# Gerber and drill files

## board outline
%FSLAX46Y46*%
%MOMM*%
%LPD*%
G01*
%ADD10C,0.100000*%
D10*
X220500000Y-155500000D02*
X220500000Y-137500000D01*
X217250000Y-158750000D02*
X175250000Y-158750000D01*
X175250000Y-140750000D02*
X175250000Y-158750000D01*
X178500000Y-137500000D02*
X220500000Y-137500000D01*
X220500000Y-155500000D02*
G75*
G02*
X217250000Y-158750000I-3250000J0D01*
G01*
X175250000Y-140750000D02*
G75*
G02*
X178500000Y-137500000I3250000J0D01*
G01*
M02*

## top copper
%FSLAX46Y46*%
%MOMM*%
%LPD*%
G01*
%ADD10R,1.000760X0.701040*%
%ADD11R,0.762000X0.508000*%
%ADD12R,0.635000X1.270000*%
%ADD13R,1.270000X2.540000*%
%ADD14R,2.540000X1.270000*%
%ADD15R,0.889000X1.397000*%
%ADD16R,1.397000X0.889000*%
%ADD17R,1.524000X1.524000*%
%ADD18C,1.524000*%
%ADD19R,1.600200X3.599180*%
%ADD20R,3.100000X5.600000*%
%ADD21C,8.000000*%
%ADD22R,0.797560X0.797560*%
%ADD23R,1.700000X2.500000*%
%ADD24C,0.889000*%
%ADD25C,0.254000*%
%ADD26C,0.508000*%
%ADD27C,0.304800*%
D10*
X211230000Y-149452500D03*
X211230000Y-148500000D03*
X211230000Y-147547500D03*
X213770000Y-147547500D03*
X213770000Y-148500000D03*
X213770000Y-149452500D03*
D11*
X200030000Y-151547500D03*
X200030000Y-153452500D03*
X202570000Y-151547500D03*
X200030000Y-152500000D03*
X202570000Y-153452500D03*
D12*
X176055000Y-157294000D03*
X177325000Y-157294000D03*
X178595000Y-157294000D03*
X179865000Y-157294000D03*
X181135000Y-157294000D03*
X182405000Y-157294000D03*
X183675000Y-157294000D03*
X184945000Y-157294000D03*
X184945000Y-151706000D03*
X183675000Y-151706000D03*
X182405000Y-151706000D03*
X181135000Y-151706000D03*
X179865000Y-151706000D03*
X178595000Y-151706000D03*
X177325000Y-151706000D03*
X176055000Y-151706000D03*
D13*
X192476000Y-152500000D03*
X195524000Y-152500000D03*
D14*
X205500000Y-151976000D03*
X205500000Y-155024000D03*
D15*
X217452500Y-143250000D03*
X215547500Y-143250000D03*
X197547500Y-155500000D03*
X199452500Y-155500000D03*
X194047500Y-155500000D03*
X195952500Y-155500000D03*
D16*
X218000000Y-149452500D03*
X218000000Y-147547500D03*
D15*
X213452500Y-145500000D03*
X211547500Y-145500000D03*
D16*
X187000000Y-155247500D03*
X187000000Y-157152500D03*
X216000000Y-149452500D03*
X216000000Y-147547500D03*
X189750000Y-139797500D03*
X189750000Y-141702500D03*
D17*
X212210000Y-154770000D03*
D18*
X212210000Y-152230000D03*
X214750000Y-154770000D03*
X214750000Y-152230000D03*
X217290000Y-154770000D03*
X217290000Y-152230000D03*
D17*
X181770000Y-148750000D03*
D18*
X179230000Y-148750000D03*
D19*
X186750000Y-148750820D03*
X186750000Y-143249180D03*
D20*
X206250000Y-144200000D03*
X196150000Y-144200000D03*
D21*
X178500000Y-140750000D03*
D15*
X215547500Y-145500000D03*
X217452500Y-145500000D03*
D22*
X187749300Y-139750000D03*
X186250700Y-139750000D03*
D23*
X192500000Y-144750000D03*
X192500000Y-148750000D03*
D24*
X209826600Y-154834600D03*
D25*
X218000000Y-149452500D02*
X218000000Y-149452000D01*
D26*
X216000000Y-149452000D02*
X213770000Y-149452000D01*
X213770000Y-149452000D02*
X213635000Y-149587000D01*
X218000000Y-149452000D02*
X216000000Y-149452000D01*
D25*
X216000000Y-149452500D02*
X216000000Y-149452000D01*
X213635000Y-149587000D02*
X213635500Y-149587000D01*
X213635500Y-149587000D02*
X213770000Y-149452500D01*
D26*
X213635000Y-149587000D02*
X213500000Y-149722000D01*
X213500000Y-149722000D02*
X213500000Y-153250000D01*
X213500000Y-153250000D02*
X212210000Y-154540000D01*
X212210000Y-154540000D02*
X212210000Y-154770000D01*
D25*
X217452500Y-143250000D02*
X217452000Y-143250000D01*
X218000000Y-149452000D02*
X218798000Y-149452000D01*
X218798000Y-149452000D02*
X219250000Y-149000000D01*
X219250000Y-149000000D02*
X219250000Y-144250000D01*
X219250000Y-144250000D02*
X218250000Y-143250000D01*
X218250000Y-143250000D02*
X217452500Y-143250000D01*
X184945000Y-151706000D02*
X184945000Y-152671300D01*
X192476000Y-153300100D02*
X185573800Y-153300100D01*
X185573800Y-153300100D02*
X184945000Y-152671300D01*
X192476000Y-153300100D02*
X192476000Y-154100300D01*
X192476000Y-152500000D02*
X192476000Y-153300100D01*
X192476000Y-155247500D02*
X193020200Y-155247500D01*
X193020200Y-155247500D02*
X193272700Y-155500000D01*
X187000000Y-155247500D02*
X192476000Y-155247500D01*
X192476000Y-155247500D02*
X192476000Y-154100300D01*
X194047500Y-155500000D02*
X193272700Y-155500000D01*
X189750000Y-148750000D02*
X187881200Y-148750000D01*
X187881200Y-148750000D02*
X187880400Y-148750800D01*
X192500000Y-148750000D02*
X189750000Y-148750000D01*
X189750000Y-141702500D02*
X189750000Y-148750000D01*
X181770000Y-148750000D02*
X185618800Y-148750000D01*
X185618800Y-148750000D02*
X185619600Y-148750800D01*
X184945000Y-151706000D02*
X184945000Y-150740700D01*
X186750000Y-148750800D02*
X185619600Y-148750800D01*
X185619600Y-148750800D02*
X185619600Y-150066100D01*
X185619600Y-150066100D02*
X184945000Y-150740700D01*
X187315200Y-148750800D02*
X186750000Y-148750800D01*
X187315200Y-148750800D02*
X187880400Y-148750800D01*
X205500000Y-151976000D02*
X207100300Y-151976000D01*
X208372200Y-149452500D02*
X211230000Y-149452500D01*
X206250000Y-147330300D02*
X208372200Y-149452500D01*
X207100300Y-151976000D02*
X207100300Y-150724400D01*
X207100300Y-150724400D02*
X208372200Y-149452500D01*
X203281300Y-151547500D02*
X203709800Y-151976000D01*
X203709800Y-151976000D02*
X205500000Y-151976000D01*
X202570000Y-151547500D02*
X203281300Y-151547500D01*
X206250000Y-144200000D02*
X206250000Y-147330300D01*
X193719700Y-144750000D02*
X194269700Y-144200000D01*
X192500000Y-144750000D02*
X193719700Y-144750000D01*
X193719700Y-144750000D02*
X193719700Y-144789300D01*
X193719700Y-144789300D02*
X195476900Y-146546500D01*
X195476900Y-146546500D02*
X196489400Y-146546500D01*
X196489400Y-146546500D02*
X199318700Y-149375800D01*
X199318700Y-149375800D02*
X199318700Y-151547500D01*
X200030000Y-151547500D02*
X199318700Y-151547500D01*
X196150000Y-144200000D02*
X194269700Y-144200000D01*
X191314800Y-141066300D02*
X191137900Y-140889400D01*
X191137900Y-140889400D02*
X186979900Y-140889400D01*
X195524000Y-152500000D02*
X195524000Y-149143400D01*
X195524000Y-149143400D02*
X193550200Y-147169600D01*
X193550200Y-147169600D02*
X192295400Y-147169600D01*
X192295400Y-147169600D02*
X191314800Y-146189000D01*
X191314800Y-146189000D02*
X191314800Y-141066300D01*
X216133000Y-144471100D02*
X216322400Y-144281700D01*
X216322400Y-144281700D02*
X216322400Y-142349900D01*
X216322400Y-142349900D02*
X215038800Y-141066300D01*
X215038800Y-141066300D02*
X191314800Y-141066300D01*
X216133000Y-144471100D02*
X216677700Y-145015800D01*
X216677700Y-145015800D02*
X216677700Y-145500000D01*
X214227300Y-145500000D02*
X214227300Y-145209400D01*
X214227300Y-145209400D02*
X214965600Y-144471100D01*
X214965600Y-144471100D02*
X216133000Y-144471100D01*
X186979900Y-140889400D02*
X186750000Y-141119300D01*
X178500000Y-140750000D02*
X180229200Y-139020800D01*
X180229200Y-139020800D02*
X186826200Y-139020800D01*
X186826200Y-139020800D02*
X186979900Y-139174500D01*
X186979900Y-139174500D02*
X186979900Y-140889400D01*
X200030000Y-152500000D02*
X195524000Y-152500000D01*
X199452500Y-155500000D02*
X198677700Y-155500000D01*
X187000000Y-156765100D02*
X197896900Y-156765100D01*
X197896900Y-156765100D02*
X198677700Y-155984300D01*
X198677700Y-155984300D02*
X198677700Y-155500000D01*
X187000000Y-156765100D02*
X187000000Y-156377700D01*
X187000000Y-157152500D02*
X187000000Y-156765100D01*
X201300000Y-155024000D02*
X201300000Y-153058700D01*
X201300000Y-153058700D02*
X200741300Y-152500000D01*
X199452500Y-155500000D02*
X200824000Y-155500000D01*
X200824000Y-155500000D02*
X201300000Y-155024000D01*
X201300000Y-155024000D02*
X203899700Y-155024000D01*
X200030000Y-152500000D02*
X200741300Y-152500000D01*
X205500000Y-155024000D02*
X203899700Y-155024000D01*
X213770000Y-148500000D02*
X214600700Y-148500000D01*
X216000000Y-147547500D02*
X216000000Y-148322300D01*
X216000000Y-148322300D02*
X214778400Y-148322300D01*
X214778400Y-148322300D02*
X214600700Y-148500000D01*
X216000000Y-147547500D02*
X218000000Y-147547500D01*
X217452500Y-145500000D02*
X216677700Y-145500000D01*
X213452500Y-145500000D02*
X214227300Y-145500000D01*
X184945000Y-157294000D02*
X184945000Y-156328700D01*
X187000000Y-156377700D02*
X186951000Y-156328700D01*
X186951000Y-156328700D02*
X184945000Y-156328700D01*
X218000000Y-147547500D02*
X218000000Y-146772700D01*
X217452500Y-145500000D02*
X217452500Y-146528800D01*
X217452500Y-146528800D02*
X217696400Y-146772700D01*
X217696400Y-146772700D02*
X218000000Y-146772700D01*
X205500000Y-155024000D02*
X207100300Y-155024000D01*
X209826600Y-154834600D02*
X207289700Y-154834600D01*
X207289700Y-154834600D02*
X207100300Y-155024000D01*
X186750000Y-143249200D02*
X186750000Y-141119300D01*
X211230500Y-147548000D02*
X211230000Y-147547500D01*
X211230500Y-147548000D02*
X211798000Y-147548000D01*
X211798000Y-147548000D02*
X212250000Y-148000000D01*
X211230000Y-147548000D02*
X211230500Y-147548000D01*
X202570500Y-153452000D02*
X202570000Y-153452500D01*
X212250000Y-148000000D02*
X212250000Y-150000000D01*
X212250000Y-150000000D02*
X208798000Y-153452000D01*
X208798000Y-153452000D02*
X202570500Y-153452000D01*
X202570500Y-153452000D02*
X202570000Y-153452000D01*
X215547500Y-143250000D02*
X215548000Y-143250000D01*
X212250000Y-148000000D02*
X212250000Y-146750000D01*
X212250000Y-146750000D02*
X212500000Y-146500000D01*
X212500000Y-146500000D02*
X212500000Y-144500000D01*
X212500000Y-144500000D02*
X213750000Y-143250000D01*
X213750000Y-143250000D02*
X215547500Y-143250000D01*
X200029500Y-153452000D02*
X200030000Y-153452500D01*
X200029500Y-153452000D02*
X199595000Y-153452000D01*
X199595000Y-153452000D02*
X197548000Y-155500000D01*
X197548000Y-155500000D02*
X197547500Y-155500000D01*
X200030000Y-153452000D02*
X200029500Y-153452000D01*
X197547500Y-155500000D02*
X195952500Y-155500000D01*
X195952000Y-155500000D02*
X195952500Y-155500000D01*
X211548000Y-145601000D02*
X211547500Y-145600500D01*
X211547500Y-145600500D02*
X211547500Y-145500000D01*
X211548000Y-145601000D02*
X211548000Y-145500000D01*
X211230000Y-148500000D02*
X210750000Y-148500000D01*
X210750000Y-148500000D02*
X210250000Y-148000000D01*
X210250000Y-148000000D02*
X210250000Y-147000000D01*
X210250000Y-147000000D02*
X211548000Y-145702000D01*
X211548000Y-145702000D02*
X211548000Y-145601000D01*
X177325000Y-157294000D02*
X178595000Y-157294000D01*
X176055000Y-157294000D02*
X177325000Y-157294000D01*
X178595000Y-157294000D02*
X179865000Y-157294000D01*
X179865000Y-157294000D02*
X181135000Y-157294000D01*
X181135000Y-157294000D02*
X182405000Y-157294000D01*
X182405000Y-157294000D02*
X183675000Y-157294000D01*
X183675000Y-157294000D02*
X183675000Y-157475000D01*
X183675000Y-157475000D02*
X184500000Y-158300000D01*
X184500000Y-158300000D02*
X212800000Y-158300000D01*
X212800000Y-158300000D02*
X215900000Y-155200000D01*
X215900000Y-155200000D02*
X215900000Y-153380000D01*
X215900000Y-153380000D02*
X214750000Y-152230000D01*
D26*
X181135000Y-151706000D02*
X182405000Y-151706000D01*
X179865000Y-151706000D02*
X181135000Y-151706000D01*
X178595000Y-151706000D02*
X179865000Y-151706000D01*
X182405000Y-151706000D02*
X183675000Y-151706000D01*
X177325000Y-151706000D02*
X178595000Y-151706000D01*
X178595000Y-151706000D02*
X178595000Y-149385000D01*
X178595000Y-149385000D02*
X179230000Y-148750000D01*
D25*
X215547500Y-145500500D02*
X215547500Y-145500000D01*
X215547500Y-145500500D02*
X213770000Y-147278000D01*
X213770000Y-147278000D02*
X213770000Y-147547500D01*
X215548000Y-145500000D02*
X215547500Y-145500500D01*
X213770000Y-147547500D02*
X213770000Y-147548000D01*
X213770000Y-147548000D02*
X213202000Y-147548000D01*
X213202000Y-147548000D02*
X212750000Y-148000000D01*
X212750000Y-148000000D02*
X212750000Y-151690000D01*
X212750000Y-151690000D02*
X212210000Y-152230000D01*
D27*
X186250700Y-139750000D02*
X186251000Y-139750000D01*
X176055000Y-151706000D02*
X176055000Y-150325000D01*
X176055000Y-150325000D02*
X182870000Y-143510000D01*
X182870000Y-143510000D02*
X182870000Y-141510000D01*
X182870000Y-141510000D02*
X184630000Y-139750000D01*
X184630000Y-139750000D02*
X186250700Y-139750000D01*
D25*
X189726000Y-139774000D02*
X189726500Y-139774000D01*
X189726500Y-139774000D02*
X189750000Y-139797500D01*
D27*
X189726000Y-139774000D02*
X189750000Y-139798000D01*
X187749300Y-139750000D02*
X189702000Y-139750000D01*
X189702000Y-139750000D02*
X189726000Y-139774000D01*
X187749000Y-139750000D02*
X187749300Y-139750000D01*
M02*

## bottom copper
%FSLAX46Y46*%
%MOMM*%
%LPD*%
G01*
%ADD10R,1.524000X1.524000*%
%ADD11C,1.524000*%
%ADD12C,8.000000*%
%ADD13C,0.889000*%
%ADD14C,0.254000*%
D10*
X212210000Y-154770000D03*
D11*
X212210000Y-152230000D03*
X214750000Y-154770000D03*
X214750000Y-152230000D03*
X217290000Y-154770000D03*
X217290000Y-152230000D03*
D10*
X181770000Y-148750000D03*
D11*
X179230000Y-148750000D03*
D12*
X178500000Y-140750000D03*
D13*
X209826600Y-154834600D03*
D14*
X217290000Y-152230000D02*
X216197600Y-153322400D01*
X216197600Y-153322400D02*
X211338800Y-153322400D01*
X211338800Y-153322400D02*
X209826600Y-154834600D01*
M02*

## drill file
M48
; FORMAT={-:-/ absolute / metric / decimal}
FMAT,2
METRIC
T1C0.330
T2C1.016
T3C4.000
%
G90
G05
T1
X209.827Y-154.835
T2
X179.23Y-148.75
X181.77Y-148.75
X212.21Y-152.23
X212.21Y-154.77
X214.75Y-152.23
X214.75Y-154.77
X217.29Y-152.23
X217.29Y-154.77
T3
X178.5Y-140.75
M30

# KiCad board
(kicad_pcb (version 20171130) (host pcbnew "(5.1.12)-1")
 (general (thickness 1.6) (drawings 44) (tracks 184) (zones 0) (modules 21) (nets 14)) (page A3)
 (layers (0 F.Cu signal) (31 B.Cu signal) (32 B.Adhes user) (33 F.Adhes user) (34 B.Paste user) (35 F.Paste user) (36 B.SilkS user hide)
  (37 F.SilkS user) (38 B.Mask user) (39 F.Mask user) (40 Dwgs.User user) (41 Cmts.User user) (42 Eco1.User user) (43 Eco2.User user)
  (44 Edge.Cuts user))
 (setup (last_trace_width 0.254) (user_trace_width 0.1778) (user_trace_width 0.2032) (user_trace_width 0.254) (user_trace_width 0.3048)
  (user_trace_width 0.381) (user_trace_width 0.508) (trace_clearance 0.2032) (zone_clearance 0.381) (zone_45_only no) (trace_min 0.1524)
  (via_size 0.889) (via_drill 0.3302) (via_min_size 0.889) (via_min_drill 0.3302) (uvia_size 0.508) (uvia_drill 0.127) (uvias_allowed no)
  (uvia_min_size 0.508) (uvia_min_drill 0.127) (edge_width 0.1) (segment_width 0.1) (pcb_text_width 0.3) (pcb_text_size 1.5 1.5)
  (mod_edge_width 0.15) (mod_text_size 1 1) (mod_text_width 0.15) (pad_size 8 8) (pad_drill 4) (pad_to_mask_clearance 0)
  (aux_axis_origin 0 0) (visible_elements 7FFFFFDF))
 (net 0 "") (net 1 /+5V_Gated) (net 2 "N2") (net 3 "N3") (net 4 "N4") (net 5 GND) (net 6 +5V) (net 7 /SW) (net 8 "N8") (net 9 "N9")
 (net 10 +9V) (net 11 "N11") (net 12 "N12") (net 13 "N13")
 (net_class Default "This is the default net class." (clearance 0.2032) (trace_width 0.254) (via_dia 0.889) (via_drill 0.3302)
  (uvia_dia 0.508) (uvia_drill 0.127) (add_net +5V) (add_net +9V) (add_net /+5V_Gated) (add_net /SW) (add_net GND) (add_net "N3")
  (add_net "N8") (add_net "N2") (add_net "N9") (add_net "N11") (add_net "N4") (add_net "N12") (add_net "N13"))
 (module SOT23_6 (layer F.Cu) (at 212.5 148.5 90)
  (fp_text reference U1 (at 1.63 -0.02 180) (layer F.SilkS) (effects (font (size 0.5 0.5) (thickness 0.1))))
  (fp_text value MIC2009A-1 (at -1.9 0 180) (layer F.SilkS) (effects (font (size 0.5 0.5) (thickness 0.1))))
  (pad 6 smd rect (at -0.9525 -1.27 90) (size 0.70104 1.00076) (layers F.Cu F.Paste F.Mask) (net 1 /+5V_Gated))
  (pad 5 smd rect (at 0 -1.27 90) (size 0.70104 1.00076) (layers F.Cu F.Paste F.Mask) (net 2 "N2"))
  (pad 4 smd rect (at 0.9525 -1.27 90) (size 0.70104 1.00076) (layers F.Cu F.Paste F.Mask) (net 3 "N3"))
  (pad 3 smd rect (at 0.9525 1.27 90) (size 0.70104 1.00076) (layers F.Cu F.Paste F.Mask) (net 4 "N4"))
  (pad 2 smd rect (at 0 1.27 90) (size 0.70104 1.00076) (layers F.Cu F.Paste F.Mask) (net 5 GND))
  (pad 1 smd rect (at -0.9525 1.27 90) (size 0.70104 1.00076) (layers F.Cu F.Paste F.Mask) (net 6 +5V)))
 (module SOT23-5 (layer F.Cu) (at 201.3 152.5 270)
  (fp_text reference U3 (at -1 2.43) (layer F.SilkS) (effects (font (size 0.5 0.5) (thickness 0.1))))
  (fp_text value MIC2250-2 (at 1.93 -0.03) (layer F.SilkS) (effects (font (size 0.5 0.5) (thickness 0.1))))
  (pad 1 smd rect (at -0.9525 1.27 270) (size 0.508 0.762) (layers F.Cu F.Paste F.Mask) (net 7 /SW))
  (pad 3 smd rect (at 0.9525 1.27 270) (size 0.508 0.762) (layers F.Cu F.Paste F.Mask) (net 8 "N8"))
  (pad 5 smd rect (at -0.9525 -1.27 270) (size 0.508 0.762) (layers F.Cu F.Paste F.Mask) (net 1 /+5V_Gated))
  (pad 2 smd rect (at 0 1.27 270) (size 0.508 0.762) (layers F.Cu F.Paste F.Mask) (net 5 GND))
  (pad 4 smd rect (at 0.9525 -1.27 270) (size 0.508 0.762) (layers F.Cu F.Paste F.Mask) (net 3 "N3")))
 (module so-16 (layer F.Cu) (at 180.5 154.5)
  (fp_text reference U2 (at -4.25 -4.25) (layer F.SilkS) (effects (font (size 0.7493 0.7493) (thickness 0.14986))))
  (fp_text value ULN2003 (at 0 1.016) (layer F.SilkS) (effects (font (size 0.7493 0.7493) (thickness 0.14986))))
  (pad 1 smd rect (at -4.445 2.794) (size 0.635 1.27) (layers F.Cu F.Paste F.Mask) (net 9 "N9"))
  (pad 2 smd rect (at -3.175 2.794) (size 0.635 1.27) (layers F.Cu F.Paste F.Mask) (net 9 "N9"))
  (pad 3 smd rect (at -1.905 2.794) (size 0.635 1.27) (layers F.Cu F.Paste F.Mask) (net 9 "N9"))
  (pad 4 smd rect (at -0.635 2.794) (size 0.635 1.27) (layers F.Cu F.Paste F.Mask) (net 9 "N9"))
  (pad 5 smd rect (at 0.635 2.794) (size 0.635 1.27) (layers F.Cu F.Paste F.Mask) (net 9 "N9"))
  (pad 6 smd rect (at 1.905 2.794) (size 0.635 1.27) (layers F.Cu F.Paste F.Mask) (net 9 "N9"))
  (pad 7 smd rect (at 3.175 2.794) (size 0.635 1.27) (layers F.Cu F.Paste F.Mask) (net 9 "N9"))
  (pad 8 smd rect (at 4.445 2.794) (size 0.635 1.27) (layers F.Cu F.Paste F.Mask) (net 5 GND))
  (pad 9 smd rect (at 4.445 -2.794) (size 0.635 1.27) (layers F.Cu F.Paste F.Mask) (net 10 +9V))
  (pad 10 smd rect (at 3.175 -2.794) (size 0.635 1.27) (layers F.Cu F.Paste F.Mask) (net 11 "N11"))
  (pad 11 smd rect (at 1.905 -2.794) (size 0.635 1.27) (layers F.Cu F.Paste F.Mask) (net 11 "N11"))
  (pad 12 smd rect (at 0.635 -2.794) (size 0.635 1.27) (layers F.Cu F.Paste F.Mask) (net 11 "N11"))
  (pad 13 smd rect (at -0.635 -2.794) (size 0.635 1.27) (layers F.Cu F.Paste F.Mask) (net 11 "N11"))
  (pad 14 smd rect (at -1.905 -2.794) (size 0.635 1.27) (layers F.Cu F.Paste F.Mask) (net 11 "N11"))
  (pad 15 smd rect (at -3.175 -2.794) (size 0.635 1.27) (layers F.Cu F.Paste F.Mask) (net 11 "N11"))
  (pad 16 smd rect (at -4.445 -2.794) (size 0.635 1.27) (layers F.Cu F.Paste F.Mask) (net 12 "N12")))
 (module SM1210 (layer F.Cu) (at 194 152.5)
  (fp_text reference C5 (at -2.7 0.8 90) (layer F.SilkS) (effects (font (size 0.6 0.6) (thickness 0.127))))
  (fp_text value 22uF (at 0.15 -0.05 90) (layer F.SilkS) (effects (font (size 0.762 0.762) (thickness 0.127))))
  (pad 1 smd rect (at -1.524 0) (size 1.27 2.54) (layers F.Cu F.Paste F.Mask) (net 10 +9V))
  (pad 2 smd rect (at 1.524 0) (size 1.27 2.54) (layers F.Cu F.Paste F.Mask) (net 5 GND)))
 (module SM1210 (layer F.Cu) (at 205.5 153.5 270)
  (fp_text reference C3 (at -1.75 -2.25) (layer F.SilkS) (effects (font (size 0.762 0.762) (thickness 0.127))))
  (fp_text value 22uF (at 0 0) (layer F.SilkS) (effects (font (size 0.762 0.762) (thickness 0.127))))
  (pad 1 smd rect (at -1.524 0 270) (size 1.27 2.54) (layers F.Cu F.Paste F.Mask) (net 1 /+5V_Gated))
  (pad 2 smd rect (at 1.524 0 270) (size 1.27 2.54) (layers F.Cu F.Paste F.Mask) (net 5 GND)))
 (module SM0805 (layer F.Cu) (at 216.5 143.25 180)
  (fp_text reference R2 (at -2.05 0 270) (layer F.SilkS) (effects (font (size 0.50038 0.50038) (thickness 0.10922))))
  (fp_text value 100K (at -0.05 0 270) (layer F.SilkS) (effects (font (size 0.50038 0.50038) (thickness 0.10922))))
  (pad 1 smd rect (at -0.9525 0 180) (size 0.889 1.397) (layers F.Cu F.Paste F.Mask) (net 6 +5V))
  (pad 2 smd rect (at 0.9525 0 180) (size 0.889 1.397) (layers F.Cu F.Paste F.Mask) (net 3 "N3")))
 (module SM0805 (layer F.Cu) (at 198.5 155.5)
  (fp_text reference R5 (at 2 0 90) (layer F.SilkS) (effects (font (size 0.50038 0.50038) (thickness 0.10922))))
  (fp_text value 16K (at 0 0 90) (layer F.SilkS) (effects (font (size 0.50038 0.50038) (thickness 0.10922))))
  (pad 1 smd rect (at -0.9525 0) (size 0.889 1.397) (layers F.Cu F.Paste F.Mask) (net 8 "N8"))
  (pad 2 smd rect (at 0.9525 0) (size 0.889 1.397) (layers F.Cu F.Paste F.Mask) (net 5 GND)))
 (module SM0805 (layer F.Cu) (at 195 155.5)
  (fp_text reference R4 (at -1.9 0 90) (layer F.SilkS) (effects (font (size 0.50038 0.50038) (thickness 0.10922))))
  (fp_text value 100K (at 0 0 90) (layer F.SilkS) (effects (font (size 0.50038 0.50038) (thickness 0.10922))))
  (pad 1 smd rect (at -0.9525 0) (size 0.889 1.397) (layers F.Cu F.Paste F.Mask) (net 10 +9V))
  (pad 2 smd rect (at 0.9525 0) (size 0.889 1.397) (layers F.Cu F.Paste F.Mask) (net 8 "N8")))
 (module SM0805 (layer F.Cu) (at 218 148.5 90)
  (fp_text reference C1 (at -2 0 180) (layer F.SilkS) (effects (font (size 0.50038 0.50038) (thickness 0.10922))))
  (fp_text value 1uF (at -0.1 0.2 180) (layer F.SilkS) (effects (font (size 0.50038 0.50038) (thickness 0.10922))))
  (pad 1 smd rect (at -0.9525 0 90) (size 0.889 1.397) (layers F.Cu F.Paste F.Mask) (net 6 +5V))
  (pad 2 smd rect (at 0.9525 0 90) (size 0.889 1.397) (layers F.Cu F.Paste F.Mask) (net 5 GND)))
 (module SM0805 (layer F.Cu) (at 212.5 145.5 180)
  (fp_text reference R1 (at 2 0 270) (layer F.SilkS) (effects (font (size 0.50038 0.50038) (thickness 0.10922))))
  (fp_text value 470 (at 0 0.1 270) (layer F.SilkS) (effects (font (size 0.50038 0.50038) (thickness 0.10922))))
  (pad 1 smd rect (at -0.9525 0 180) (size 0.889 1.397) (layers F.Cu F.Paste F.Mask) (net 5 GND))
  (pad 2 smd rect (at 0.9525 0 180) (size 0.889 1.397) (layers F.Cu F.Paste F.Mask) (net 2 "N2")))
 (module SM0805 (layer F.Cu) (at 187 156.2 270)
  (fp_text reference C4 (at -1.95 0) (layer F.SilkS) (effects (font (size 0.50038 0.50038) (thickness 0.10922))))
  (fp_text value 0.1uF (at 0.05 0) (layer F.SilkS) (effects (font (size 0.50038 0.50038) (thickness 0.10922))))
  (pad 1 smd rect (at -0.9525 0 270) (size 0.889 1.397) (layers F.Cu F.Paste F.Mask) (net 10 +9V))
  (pad 2 smd rect (at 0.9525 0 270) (size 0.889 1.397) (layers F.Cu F.Paste F.Mask) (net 5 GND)))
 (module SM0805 (layer F.Cu) (at 216 148.5 90)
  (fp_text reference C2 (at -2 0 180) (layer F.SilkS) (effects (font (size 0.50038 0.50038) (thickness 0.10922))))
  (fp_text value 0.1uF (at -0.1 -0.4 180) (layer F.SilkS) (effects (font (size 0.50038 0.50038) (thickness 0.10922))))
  (pad 1 smd rect (at -0.9525 0 90) (size 0.889 1.397) (layers F.Cu F.Paste F.Mask) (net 6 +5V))
  (pad 2 smd rect (at 0.9525 0 90) (size 0.889 1.397) (layers F.Cu F.Paste F.Mask) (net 5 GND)))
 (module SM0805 (layer F.Cu) (at 189.75 140.75 270)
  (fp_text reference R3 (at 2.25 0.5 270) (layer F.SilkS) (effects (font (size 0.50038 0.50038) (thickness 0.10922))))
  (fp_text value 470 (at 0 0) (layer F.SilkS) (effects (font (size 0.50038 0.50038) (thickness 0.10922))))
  (pad 1 smd rect (at -0.9525 0 270) (size 0.889 1.397) (layers F.Cu F.Paste F.Mask) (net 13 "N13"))
  (pad 2 smd rect (at 0.9525 0 270) (size 0.889 1.397) (layers F.Cu F.Paste F.Mask) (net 10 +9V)))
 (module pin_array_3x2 (layer F.Cu) (at 214.75 153.5)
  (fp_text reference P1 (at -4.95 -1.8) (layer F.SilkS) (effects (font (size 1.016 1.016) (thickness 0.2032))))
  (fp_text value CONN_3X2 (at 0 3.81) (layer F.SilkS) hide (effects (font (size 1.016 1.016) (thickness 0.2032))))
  (pad 1 thru_hole rect (at -2.54 1.27) (size 1.524 1.524) (drill 1.016) (layers *.Cu *.Mask F.SilkS) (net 6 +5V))
  (pad 2 thru_hole circle (at -2.54 -1.27) (size 1.524 1.524) (drill 1.016) (layers *.Cu *.Mask F.SilkS) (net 4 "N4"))
  (pad 3 thru_hole circle (at 0 1.27) (size 1.524 1.524) (drill 1.016) (layers *.Cu *.Mask F.SilkS))
  (pad 4 thru_hole circle (at 0 -1.27) (size 1.524 1.524) (drill 1.016) (layers *.Cu *.Mask F.SilkS) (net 9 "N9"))
  (pad 5 thru_hole circle (at 2.54 1.27) (size 1.524 1.524) (drill 1.016) (layers *.Cu *.Mask F.SilkS))
  (pad 6 thru_hole circle (at 2.54 -1.27) (size 1.524 1.524) (drill 1.016) (layers *.Cu *.Mask F.SilkS) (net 5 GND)))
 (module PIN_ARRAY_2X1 (layer F.Cu) (at 180.5 148.75 180)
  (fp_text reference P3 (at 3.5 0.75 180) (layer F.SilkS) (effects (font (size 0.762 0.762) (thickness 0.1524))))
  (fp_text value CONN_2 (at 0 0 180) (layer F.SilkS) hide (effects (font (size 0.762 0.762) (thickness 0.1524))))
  (pad 1 thru_hole rect (at -1.27 0 180) (size 1.524 1.524) (drill 1.016) (layers *.Cu *.Mask F.SilkS) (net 10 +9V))
  (pad 2 thru_hole circle (at 1.27 0 180) (size 1.524 1.524) (drill 1.016) (layers *.Cu *.Mask F.SilkS) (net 11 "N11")))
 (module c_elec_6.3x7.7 (layer F.Cu) (at 186.75 146 270)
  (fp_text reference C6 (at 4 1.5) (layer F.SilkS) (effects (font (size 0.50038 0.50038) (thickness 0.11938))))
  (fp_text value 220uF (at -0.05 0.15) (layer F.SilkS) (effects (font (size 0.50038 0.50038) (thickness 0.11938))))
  (pad 1 smd rect (at 2.75082 0 270) (size 3.59918 1.6002) (layers F.Cu F.Paste F.Mask) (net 10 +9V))
  (pad 2 smd rect (at -2.75082 0 270) (size 3.59918 1.6002) (layers F.Cu F.Paste F.Mask) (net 5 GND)))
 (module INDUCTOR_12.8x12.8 (layer F.Cu) (at 201.2 144.2 180)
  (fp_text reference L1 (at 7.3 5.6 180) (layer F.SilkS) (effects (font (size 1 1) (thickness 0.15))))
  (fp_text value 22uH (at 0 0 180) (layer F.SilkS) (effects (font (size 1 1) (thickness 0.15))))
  (pad 1 smd rect (at -5.05 0 180) (size 3.1 5.6) (layers F.Cu F.Paste F.Mask) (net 1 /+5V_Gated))
  (pad 2 smd rect (at 5.05 0 180) (size 3.1 5.6) (layers F.Cu F.Paste F.Mask) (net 7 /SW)))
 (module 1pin (layer F.Cu) (at 178.5 140.75)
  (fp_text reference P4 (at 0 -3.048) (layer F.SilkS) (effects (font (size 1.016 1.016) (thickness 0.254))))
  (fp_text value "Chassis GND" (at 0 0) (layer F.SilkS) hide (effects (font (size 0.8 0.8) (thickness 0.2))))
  (pad 1 thru_hole circle (at 0 0) (size 8 8) (drill 4) (layers *.Cu *.Mask F.SilkS) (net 5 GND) (zone_connect 2)))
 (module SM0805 (layer F.Cu) (at 216.5 145.5)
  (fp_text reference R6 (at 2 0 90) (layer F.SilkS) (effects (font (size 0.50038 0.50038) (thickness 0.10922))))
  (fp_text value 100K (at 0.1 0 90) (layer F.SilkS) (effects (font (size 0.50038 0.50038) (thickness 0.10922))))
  (pad 1 smd rect (at -0.9525 0) (size 0.889 1.397) (layers F.Cu F.Paste F.Mask) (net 4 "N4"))
  (pad 2 smd rect (at 0.9525 0) (size 0.889 1.397) (layers F.Cu F.Paste F.Mask) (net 5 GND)))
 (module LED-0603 (layer F.Cu) (at 187 139.75 180)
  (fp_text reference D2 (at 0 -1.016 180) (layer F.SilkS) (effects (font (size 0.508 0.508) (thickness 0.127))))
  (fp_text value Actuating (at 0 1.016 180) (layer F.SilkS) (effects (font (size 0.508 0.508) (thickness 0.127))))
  (pad 1 smd rect (at -0.7493 0 180) (size 0.79756 0.79756) (layers F.Cu F.Paste F.Mask) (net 13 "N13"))
  (pad 2 smd rect (at 0.7493 0 180) (size 0.79756 0.79756) (layers F.Cu F.Paste F.Mask) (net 12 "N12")))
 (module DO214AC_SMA (layer F.Cu) (at 192.5 146.75 270)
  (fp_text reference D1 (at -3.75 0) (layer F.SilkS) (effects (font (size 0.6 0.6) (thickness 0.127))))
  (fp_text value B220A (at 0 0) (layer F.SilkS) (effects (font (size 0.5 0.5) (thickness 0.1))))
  (pad 1 smd rect (at -2 0 270) (size 2.5 1.7) (layers F.Cu F.Paste F.Mask) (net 7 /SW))
  (pad 2 smd rect (at 2 0 270) (size 2.5 1.7) (layers F.Cu F.Paste F.Mask) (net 10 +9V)))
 (gr_line (start 220.5 155.5) (end 220.5 137.5) (angle 90) (layer Edge.Cuts) (width 0.1))
 (gr_line (start 217.25 158.75) (end 175.25 158.75) (angle 90) (layer Edge.Cuts) (width 0.1))
 (gr_line (start 175.25 140.75) (end 175.25 158.75) (angle 90) (layer Edge.Cuts) (width 0.1))
 (gr_line (start 178.5 137.5) (end 220.5 137.5) (angle 90) (layer Edge.Cuts) (width 0.1))
 (gr_arc (start 217.25 155.5) (end 220.5 155.5) (angle 90) (layer Edge.Cuts) (width 0.1))
 (gr_arc (start 178.5 140.75) (end 175.25 140.75) (angle 90) (layer Edge.Cuts) (width 0.1))
 (segment (start 218 149.4525) (end 218 149.452) (width 0.254) (layer F.Cu) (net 6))
 (segment (start 216 149.452) (end 213.77 149.452) (width 0.508) (layer F.Cu) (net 6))
 (segment (start 213.77 149.452) (end 213.635 149.587) (width 0.508) (layer F.Cu) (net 6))
 (segment (start 218 149.452) (end 216 149.452) (width 0.508) (layer F.Cu) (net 6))
 (segment (start 216 149.4525) (end 216 149.452) (width 0.254) (layer F.Cu) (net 6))
 (segment (start 213.635 149.587) (end 213.6355 149.587) (width 0.254) (layer F.Cu) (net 6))
 (segment (start 213.6355 149.587) (end 213.77 149.4525) (width 0.254) (layer F.Cu) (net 6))
 (segment (start 213.635 149.587) (end 213.5 149.722) (width 0.508) (layer F.Cu) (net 6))
 (segment (start 213.5 149.722) (end 213.5 153.25) (width 0.508) (layer F.Cu) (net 6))
 (segment (start 213.5 153.25) (end 212.21 154.54) (width 0.508) (layer F.Cu) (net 6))
 (segment (start 212.21 154.54) (end 212.21 154.77) (width 0.508) (layer F.Cu) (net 6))
 (segment (start 217.4525 143.25) (end 217.452 143.25) (width 0.254) (layer F.Cu) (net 6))
 (segment (start 218 149.452) (end 218.798 149.452) (width 0.254) (layer F.Cu) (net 6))
 (segment (start 218.798 149.452) (end 219.25 149) (width 0.254) (layer F.Cu) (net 6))
 (segment (start 219.25 149) (end 219.25 144.25) (width 0.254) (layer F.Cu) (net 6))
 (segment (start 219.25 144.25) (end 218.25 143.25) (width 0.254) (layer F.Cu) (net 6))
 (segment (start 218.25 143.25) (end 217.4525 143.25) (width 0.254) (layer F.Cu) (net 6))
 (segment (start 184.945 151.706) (end 184.945 152.6713) (width 0.254) (layer F.Cu) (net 10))
 (segment (start 192.476 153.3001) (end 185.5738 153.3001) (width 0.254) (layer F.Cu) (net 10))
 (segment (start 185.5738 153.3001) (end 184.945 152.6713) (width 0.254) (layer F.Cu) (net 10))
 (segment (start 192.476 153.3001) (end 192.476 154.1003) (width 0.254) (layer F.Cu) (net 10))
 (segment (start 192.476 152.5) (end 192.476 153.3001) (width 0.254) (layer F.Cu) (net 10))
 (segment (start 192.476 155.2475) (end 193.0202 155.2475) (width 0.254) (layer F.Cu) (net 10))
 (segment (start 193.0202 155.2475) (end 193.2727 155.5) (width 0.254) (layer F.Cu) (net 10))
 (segment (start 187 155.2475) (end 192.476 155.2475) (width 0.254) (layer F.Cu) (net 10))
 (segment (start 192.476 155.2475) (end 192.476 154.1003) (width 0.254) (layer F.Cu) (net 10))
 (segment (start 194.0475 155.5) (end 193.2727 155.5) (width 0.254) (layer F.Cu) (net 10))
 (segment (start 189.75 148.75) (end 187.8812 148.75) (width 0.254) (layer F.Cu) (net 10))
 (segment (start 187.8812 148.75) (end 187.8804 148.7508) (width 0.254) (layer F.Cu) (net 10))
 (segment (start 192.5 148.75) (end 189.75 148.75) (width 0.254) (layer F.Cu) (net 10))
 (segment (start 189.75 141.7025) (end 189.75 148.75) (width 0.254) (layer F.Cu) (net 10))
 (segment (start 181.77 148.75) (end 185.6188 148.75) (width 0.254) (layer F.Cu) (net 10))
 (segment (start 185.6188 148.75) (end 185.6196 148.7508) (width 0.254) (layer F.Cu) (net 10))
 (segment (start 184.945 151.706) (end 184.945 150.7407) (width 0.254) (layer F.Cu) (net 10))
 (segment (start 186.75 148.7508) (end 185.6196 148.7508) (width 0.254) (layer F.Cu) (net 10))
 (segment (start 185.6196 148.7508) (end 185.6196 150.0661) (width 0.254) (layer F.Cu) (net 10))
 (segment (start 185.6196 150.0661) (end 184.945 150.7407) (width 0.254) (layer F.Cu) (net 10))
 (segment (start 187.3152 148.7508) (end 186.75 148.7508) (width 0.254) (layer F.Cu) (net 10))
 (segment (start 187.3152 148.7508) (end 187.8804 148.7508) (width 0.254) (layer F.Cu) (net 10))
 (segment (start 205.5 151.976) (end 207.1003 151.976) (width 0.254) (layer F.Cu) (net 1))
 (segment (start 208.3722 149.4525) (end 211.23 149.4525) (width 0.254) (layer F.Cu) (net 1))
 (segment (start 206.25 147.3303) (end 208.3722 149.4525) (width 0.254) (layer F.Cu) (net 1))
 (segment (start 207.1003 151.976) (end 207.1003 150.7244) (width 0.254) (layer F.Cu) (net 1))
 (segment (start 207.1003 150.7244) (end 208.3722 149.4525) (width 0.254) (layer F.Cu) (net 1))
 (segment (start 203.2813 151.5475) (end 203.7098 151.976) (width 0.254) (layer F.Cu) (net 1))
 (segment (start 203.7098 151.976) (end 205.5 151.976) (width 0.254) (layer F.Cu) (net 1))
 (segment (start 202.57 151.5475) (end 203.2813 151.5475) (width 0.254) (layer F.Cu) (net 1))
 (segment (start 206.25 144.2) (end 206.25 147.3303) (width 0.254) (layer F.Cu) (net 1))
 (segment (start 193.7197 144.75) (end 194.2697 144.2) (width 0.254) (layer F.Cu) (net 7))
 (segment (start 192.5 144.75) (end 193.7197 144.75) (width 0.254) (layer F.Cu) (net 7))
 (segment (start 193.7197 144.75) (end 193.7197 144.7893) (width 0.254) (layer F.Cu) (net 7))
 (segment (start 193.7197 144.7893) (end 195.4769 146.5465) (width 0.254) (layer F.Cu) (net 7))
 (segment (start 195.4769 146.5465) (end 196.4894 146.5465) (width 0.254) (layer F.Cu) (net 7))
 (segment (start 196.4894 146.5465) (end 199.3187 149.3758) (width 0.254) (layer F.Cu) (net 7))
 (segment (start 199.3187 149.3758) (end 199.3187 151.5475) (width 0.254) (layer F.Cu) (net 7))
 (segment (start 200.03 151.5475) (end 199.3187 151.5475) (width 0.254) (layer F.Cu) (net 7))
 (segment (start 196.15 144.2) (end 194.2697 144.2) (width 0.254) (layer F.Cu) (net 7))
 (segment (start 191.3148 141.0663) (end 191.1379 140.8894) (width 0.254) (layer F.Cu) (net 5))
 (segment (start 191.1379 140.8894) (end 186.9799 140.8894) (width 0.254) (layer F.Cu) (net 5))
 (segment (start 195.524 152.5) (end 195.524 149.1434) (width 0.254) (layer F.Cu) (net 5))
 (segment (start 195.524 149.1434) (end 193.5502 147.1696) (width 0.254) (layer F.Cu) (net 5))
 (segment (start 193.5502 147.1696) (end 192.2954 147.1696) (width 0.254) (layer F.Cu) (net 5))
 (segment (start 192.2954 147.1696) (end 191.3148 146.189) (width 0.254) (layer F.Cu) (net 5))
 (segment (start 191.3148 146.189) (end 191.3148 141.0663) (width 0.254) (layer F.Cu) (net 5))
 (segment (start 216.133 144.4711) (end 216.3224 144.2817) (width 0.254) (layer F.Cu) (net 5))
 (segment (start 216.3224 144.2817) (end 216.3224 142.3499) (width 0.254) (layer F.Cu) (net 5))
 (segment (start 216.3224 142.3499) (end 215.0388 141.0663) (width 0.254) (layer F.Cu) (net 5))
 (segment (start 215.0388 141.0663) (end 191.3148 141.0663) (width 0.254) (layer F.Cu) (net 5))
 (segment (start 216.133 144.4711) (end 216.6777 145.0158) (width 0.254) (layer F.Cu) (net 5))
 (segment (start 216.6777 145.0158) (end 216.6777 145.5) (width 0.254) (layer F.Cu) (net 5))
 (segment (start 214.2273 145.5) (end 214.2273 145.2094) (width 0.254) (layer F.Cu) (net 5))
 (segment (start 214.2273 145.2094) (end 214.9656 144.4711) (width 0.254) (layer F.Cu) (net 5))
 (segment (start 214.9656 144.4711) (end 216.133 144.4711) (width 0.254) (layer F.Cu) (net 5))
 (segment (start 186.9799 140.8894) (end 186.75 141.1193) (width 0.254) (layer F.Cu) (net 5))
 (segment (start 178.5 140.75) (end 180.2292 139.0208) (width 0.254) (layer F.Cu) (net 5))
 (segment (start 180.2292 139.0208) (end 186.8262 139.0208) (width 0.254) (layer F.Cu) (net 5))
 (segment (start 186.8262 139.0208) (end 186.9799 139.1745) (width 0.254) (layer F.Cu) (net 5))
 (segment (start 186.9799 139.1745) (end 186.9799 140.8894) (width 0.254) (layer F.Cu) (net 5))
 (segment (start 200.03 152.5) (end 195.524 152.5) (width 0.254) (layer F.Cu) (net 5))
 (segment (start 199.4525 155.5) (end 198.6777 155.5) (width 0.254) (layer F.Cu) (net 5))
 (segment (start 187 156.7651) (end 197.8969 156.7651) (width 0.254) (layer F.Cu) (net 5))
 (segment (start 197.8969 156.7651) (end 198.6777 155.9843) (width 0.254) (layer F.Cu) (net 5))
 (segment (start 198.6777 155.9843) (end 198.6777 155.5) (width 0.254) (layer F.Cu) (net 5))
 (segment (start 187 156.7651) (end 187 156.3777) (width 0.254) (layer F.Cu) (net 5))
 (segment (start 187 157.1525) (end 187 156.7651) (width 0.254) (layer F.Cu) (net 5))
 (segment (start 201.3 155.024) (end 201.3 153.0587) (width 0.254) (layer F.Cu) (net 5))
 (segment (start 201.3 153.0587) (end 200.7413 152.5) (width 0.254) (layer F.Cu) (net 5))
 (segment (start 199.4525 155.5) (end 200.824 155.5) (width 0.254) (layer F.Cu) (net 5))
 (segment (start 200.824 155.5) (end 201.3 155.024) (width 0.254) (layer F.Cu) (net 5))
 (segment (start 201.3 155.024) (end 203.8997 155.024) (width 0.254) (layer F.Cu) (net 5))
 (segment (start 200.03 152.5) (end 200.7413 152.5) (width 0.254) (layer F.Cu) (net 5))
 (segment (start 205.5 155.024) (end 203.8997 155.024) (width 0.254) (layer F.Cu) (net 5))
 (segment (start 213.77 148.5) (end 214.6007 148.5) (width 0.254) (layer F.Cu) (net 5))
 (segment (start 216 147.5475) (end 216 148.3223) (width 0.254) (layer F.Cu) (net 5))
 (segment (start 216 148.3223) (end 214.7784 148.3223) (width 0.254) (layer F.Cu) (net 5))
 (segment (start 214.7784 148.3223) (end 214.6007 148.5) (width 0.254) (layer F.Cu) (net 5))
 (segment (start 216 147.5475) (end 218 147.5475) (width 0.254) (layer F.Cu) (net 5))
 (segment (start 217.4525 145.5) (end 216.6777 145.5) (width 0.254) (layer F.Cu) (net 5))
 (segment (start 213.4525 145.5) (end 214.2273 145.5) (width 0.254) (layer F.Cu) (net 5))
 (segment (start 184.945 157.294) (end 184.945 156.3287) (width 0.254) (layer F.Cu) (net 5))
 (segment (start 187 156.3777) (end 186.951 156.3287) (width 0.254) (layer F.Cu) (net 5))
 (segment (start 186.951 156.3287) (end 184.945 156.3287) (width 0.254) (layer F.Cu) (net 5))
 (segment (start 218 147.5475) (end 218 146.7727) (width 0.254) (layer F.Cu) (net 5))
 (segment (start 217.4525 145.5) (end 217.4525 146.5288) (width 0.254) (layer F.Cu) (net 5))
 (segment (start 217.4525 146.5288) (end 217.6964 146.7727) (width 0.254) (layer F.Cu) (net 5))
 (segment (start 217.6964 146.7727) (end 218 146.7727) (width 0.254) (layer F.Cu) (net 5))
 (segment (start 205.5 155.024) (end 207.1003 155.024) (width 0.254) (layer F.Cu) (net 5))
 (segment (start 209.8266 154.8346) (end 207.2897 154.8346) (width 0.254) (layer F.Cu) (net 5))
 (segment (start 207.2897 154.8346) (end 207.1003 155.024) (width 0.254) (layer F.Cu) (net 5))
 (segment (start 217.29 152.23) (end 216.1976 153.3224) (width 0.254) (layer B.Cu) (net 5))
 (segment (start 216.1976 153.3224) (end 211.3388 153.3224) (width 0.254) (layer B.Cu) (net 5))
 (segment (start 211.3388 153.3224) (end 209.8266 154.8346) (width 0.254) (layer B.Cu) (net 5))
 (segment (start 186.75 143.2492) (end 186.75 141.1193) (width 0.254) (layer F.Cu) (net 5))
 (via (at 209.8266 154.8346) (size 0.889) (layers F.Cu B.Cu) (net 5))
 (segment (start 211.2305 147.548) (end 211.23 147.5475) (width 0.254) (layer F.Cu) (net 3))
 (segment (start 211.2305 147.548) (end 211.798 147.548) (width 0.254) (layer F.Cu) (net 3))
 (segment (start 211.798 147.548) (end 212.25 148) (width 0.254) (layer F.Cu) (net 3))
 (segment (start 211.23 147.548) (end 211.2305 147.548) (width 0.254) (layer F.Cu) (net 3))
 (segment (start 202.5705 153.452) (end 202.57 153.4525) (width 0.254) (layer F.Cu) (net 3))
 (segment (start 212.25 148) (end 212.25 150) (width 0.254) (layer F.Cu) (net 3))
 (segment (start 212.25 150) (end 208.798 153.452) (width 0.254) (layer F.Cu) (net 3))
 (segment (start 208.798 153.452) (end 202.5705 153.452) (width 0.254) (layer F.Cu) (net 3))
 (segment (start 202.5705 153.452) (end 202.57 153.452) (width 0.254) (layer F.Cu) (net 3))
 (segment (start 215.5475 143.25) (end 215.548 143.25) (width 0.254) (layer F.Cu) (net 3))
 (segment (start 212.25 148) (end 212.25 146.75) (width 0.254) (layer F.Cu) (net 3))
 (segment (start 212.25 146.75) (end 212.5 146.5) (width 0.254) (layer F.Cu) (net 3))
 (segment (start 212.5 146.5) (end 212.5 144.5) (width 0.254) (layer F.Cu) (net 3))
 (segment (start 212.5 144.5) (end 213.75 143.25) (width 0.254) (layer F.Cu) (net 3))
 (segment (start 213.75 143.25) (end 215.5475 143.25) (width 0.254) (layer F.Cu) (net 3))
 (segment (start 200.0295 153.452) (end 200.03 153.4525) (width 0.254) (layer F.Cu) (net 8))
 (segment (start 200.0295 153.452) (end 199.595 153.452) (width 0.254) (layer F.Cu) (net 8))
 (segment (start 199.595 153.452) (end 197.548 155.5) (width 0.254) (layer F.Cu) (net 8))
 (segment (start 197.548 155.5) (end 197.5475 155.5) (width 0.254) (layer F.Cu) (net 8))
 (segment (start 200.03 153.452) (end 200.0295 153.452) (width 0.254) (layer F.Cu) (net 8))
 (segment (start 197.5475 155.5) (end 195.9525 155.5) (width 0.254) (layer F.Cu) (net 8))
 (segment (start 195.952 155.5) (end 195.9525 155.5) (width 0.254) (layer F.Cu) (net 8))
 (segment (start 211.548 145.601) (end 211.5475 145.6005) (width 0.254) (layer F.Cu) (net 2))
 (segment (start 211.5475 145.6005) (end 211.5475 145.5) (width 0.254) (layer F.Cu) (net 2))
 (segment (start 211.548 145.601) (end 211.548 145.5) (width 0.254) (layer F.Cu) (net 2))
 (segment (start 211.23 148.5) (end 210.75 148.5) (width 0.254) (layer F.Cu) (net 2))
 (segment (start 210.75 148.5) (end 210.25 148) (width 0.254) (layer F.Cu) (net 2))
 (segment (start 210.25 148) (end 210.25 147) (width 0.254) (layer F.Cu) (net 2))
 (segment (start 210.25 147) (end 211.548 145.702) (width 0.254) (layer F.Cu) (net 2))
 (segment (start 211.548 145.702) (end 211.548 145.601) (width 0.254) (layer F.Cu) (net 2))
 (segment (start 177.325 157.294) (end 178.595 157.294) (width 0.254) (layer F.Cu) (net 9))
 (segment (start 176.055 157.294) (end 177.325 157.294) (width 0.254) (layer F.Cu) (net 9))
 (segment (start 178.595 157.294) (end 179.865 157.294) (width 0.254) (layer F.Cu) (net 9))
 (segment (start 179.865 157.294) (end 181.135 157.294) (width 0.254) (layer F.Cu) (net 9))
 (segment (start 181.135 157.294) (end 182.405 157.294) (width 0.254) (layer F.Cu) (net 9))
 (segment (start 182.405 157.294) (end 183.675 157.294) (width 0.254) (layer F.Cu) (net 9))
 (segment (start 183.675 157.294) (end 183.675 157.475) (width 0.254) (layer F.Cu) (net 9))
 (segment (start 183.675 157.475) (end 184.5 158.3) (width 0.254) (layer F.Cu) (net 9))
 (segment (start 184.5 158.3) (end 212.8 158.3) (width 0.254) (layer F.Cu) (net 9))
 (segment (start 212.8 158.3) (end 215.9 155.2) (width 0.254) (layer F.Cu) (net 9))
 (segment (start 215.9 155.2) (end 215.9 153.38) (width 0.254) (layer F.Cu) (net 9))
 (segment (start 215.9 153.38) (end 214.75 152.23) (width 0.254) (layer F.Cu) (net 9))
 (segment (start 181.135 151.706) (end 182.405 151.706) (width 0.508) (layer F.Cu) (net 11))
 (segment (start 179.865 151.706) (end 181.135 151.706) (width 0.508) (layer F.Cu) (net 11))
 (segment (start 178.595 151.706) (end 179.865 151.706) (width 0.508) (layer F.Cu) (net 11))
 (segment (start 182.405 151.706) (end 183.675 151.706) (width 0.508) (layer F.Cu) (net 11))
 (segment (start 177.325 151.706) (end 178.595 151.706) (width 0.508) (layer F.Cu) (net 11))
 (segment (start 178.595 151.706) (end 178.595 149.385) (width 0.508) (layer F.Cu) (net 11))
 (segment (start 178.595 149.385) (end 179.23 148.75) (width 0.508) (layer F.Cu) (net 11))
 (segment (start 215.5475 145.5005) (end 215.5475 145.5) (width 0.254) (layer F.Cu) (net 4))
 (segment (start 215.5475 145.5005) (end 213.77 147.278) (width 0.254) (layer F.Cu) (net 4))
 (segment (start 213.77 147.278) (end 213.77 147.5475) (width 0.254) (layer F.Cu) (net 4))
 (segment (start 215.548 145.5) (end 215.5475 145.5005) (width 0.254) (layer F.Cu) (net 4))
 (segment (start 213.77 147.5475) (end 213.77 147.548) (width 0.254) (layer F.Cu) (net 4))
 (segment (start 213.77 147.548) (end 213.202 147.548) (width 0.254) (layer F.Cu) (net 4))
 (segment (start 213.202 147.548) (end 212.75 148) (width 0.254) (layer F.Cu) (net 4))
 (segment (start 212.75 148) (end 212.75 151.69) (width 0.254) (layer F.Cu) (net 4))
 (segment (start 212.75 151.69) (end 212.21 152.23) (width 0.254) (layer F.Cu) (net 4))
 (segment (start 186.2507 139.75) (end 186.251 139.75) (width 0.3048) (layer F.Cu) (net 12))
 (segment (start 176.055 151.706) (end 176.055 150.325) (width 0.3048) (layer F.Cu) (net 12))
 (segment (start 176.055 150.325) (end 182.87 143.51) (width 0.3048) (layer F.Cu) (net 12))
 (segment (start 182.87 143.51) (end 182.87 141.51) (width 0.3048) (layer F.Cu) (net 12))
 (segment (start 182.87 141.51) (end 184.63 139.75) (width 0.3048) (layer F.Cu) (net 12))
 (segment (start 184.63 139.75) (end 186.2507 139.75) (width 0.3048) (layer F.Cu) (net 12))
 (segment (start 189.726 139.774) (end 189.7265 139.774) (width 0.254) (layer F.Cu) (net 13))
 (segment (start 189.7265 139.774) (end 189.75 139.7975) (width 0.254) (layer F.Cu) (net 13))
 (segment (start 189.726 139.774) (end 189.75 139.798) (width 0.3048) (layer F.Cu) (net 13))
 (segment (start 187.7493 139.75) (end 189.702 139.75) (width 0.3048) (layer F.Cu) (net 13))
 (segment (start 189.702 139.75) (end 189.726 139.774) (width 0.3048) (layer F.Cu) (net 13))
 (segment (start 187.749 139.75) (end 187.7493 139.75) (width 0.3048) (layer F.Cu) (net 13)))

